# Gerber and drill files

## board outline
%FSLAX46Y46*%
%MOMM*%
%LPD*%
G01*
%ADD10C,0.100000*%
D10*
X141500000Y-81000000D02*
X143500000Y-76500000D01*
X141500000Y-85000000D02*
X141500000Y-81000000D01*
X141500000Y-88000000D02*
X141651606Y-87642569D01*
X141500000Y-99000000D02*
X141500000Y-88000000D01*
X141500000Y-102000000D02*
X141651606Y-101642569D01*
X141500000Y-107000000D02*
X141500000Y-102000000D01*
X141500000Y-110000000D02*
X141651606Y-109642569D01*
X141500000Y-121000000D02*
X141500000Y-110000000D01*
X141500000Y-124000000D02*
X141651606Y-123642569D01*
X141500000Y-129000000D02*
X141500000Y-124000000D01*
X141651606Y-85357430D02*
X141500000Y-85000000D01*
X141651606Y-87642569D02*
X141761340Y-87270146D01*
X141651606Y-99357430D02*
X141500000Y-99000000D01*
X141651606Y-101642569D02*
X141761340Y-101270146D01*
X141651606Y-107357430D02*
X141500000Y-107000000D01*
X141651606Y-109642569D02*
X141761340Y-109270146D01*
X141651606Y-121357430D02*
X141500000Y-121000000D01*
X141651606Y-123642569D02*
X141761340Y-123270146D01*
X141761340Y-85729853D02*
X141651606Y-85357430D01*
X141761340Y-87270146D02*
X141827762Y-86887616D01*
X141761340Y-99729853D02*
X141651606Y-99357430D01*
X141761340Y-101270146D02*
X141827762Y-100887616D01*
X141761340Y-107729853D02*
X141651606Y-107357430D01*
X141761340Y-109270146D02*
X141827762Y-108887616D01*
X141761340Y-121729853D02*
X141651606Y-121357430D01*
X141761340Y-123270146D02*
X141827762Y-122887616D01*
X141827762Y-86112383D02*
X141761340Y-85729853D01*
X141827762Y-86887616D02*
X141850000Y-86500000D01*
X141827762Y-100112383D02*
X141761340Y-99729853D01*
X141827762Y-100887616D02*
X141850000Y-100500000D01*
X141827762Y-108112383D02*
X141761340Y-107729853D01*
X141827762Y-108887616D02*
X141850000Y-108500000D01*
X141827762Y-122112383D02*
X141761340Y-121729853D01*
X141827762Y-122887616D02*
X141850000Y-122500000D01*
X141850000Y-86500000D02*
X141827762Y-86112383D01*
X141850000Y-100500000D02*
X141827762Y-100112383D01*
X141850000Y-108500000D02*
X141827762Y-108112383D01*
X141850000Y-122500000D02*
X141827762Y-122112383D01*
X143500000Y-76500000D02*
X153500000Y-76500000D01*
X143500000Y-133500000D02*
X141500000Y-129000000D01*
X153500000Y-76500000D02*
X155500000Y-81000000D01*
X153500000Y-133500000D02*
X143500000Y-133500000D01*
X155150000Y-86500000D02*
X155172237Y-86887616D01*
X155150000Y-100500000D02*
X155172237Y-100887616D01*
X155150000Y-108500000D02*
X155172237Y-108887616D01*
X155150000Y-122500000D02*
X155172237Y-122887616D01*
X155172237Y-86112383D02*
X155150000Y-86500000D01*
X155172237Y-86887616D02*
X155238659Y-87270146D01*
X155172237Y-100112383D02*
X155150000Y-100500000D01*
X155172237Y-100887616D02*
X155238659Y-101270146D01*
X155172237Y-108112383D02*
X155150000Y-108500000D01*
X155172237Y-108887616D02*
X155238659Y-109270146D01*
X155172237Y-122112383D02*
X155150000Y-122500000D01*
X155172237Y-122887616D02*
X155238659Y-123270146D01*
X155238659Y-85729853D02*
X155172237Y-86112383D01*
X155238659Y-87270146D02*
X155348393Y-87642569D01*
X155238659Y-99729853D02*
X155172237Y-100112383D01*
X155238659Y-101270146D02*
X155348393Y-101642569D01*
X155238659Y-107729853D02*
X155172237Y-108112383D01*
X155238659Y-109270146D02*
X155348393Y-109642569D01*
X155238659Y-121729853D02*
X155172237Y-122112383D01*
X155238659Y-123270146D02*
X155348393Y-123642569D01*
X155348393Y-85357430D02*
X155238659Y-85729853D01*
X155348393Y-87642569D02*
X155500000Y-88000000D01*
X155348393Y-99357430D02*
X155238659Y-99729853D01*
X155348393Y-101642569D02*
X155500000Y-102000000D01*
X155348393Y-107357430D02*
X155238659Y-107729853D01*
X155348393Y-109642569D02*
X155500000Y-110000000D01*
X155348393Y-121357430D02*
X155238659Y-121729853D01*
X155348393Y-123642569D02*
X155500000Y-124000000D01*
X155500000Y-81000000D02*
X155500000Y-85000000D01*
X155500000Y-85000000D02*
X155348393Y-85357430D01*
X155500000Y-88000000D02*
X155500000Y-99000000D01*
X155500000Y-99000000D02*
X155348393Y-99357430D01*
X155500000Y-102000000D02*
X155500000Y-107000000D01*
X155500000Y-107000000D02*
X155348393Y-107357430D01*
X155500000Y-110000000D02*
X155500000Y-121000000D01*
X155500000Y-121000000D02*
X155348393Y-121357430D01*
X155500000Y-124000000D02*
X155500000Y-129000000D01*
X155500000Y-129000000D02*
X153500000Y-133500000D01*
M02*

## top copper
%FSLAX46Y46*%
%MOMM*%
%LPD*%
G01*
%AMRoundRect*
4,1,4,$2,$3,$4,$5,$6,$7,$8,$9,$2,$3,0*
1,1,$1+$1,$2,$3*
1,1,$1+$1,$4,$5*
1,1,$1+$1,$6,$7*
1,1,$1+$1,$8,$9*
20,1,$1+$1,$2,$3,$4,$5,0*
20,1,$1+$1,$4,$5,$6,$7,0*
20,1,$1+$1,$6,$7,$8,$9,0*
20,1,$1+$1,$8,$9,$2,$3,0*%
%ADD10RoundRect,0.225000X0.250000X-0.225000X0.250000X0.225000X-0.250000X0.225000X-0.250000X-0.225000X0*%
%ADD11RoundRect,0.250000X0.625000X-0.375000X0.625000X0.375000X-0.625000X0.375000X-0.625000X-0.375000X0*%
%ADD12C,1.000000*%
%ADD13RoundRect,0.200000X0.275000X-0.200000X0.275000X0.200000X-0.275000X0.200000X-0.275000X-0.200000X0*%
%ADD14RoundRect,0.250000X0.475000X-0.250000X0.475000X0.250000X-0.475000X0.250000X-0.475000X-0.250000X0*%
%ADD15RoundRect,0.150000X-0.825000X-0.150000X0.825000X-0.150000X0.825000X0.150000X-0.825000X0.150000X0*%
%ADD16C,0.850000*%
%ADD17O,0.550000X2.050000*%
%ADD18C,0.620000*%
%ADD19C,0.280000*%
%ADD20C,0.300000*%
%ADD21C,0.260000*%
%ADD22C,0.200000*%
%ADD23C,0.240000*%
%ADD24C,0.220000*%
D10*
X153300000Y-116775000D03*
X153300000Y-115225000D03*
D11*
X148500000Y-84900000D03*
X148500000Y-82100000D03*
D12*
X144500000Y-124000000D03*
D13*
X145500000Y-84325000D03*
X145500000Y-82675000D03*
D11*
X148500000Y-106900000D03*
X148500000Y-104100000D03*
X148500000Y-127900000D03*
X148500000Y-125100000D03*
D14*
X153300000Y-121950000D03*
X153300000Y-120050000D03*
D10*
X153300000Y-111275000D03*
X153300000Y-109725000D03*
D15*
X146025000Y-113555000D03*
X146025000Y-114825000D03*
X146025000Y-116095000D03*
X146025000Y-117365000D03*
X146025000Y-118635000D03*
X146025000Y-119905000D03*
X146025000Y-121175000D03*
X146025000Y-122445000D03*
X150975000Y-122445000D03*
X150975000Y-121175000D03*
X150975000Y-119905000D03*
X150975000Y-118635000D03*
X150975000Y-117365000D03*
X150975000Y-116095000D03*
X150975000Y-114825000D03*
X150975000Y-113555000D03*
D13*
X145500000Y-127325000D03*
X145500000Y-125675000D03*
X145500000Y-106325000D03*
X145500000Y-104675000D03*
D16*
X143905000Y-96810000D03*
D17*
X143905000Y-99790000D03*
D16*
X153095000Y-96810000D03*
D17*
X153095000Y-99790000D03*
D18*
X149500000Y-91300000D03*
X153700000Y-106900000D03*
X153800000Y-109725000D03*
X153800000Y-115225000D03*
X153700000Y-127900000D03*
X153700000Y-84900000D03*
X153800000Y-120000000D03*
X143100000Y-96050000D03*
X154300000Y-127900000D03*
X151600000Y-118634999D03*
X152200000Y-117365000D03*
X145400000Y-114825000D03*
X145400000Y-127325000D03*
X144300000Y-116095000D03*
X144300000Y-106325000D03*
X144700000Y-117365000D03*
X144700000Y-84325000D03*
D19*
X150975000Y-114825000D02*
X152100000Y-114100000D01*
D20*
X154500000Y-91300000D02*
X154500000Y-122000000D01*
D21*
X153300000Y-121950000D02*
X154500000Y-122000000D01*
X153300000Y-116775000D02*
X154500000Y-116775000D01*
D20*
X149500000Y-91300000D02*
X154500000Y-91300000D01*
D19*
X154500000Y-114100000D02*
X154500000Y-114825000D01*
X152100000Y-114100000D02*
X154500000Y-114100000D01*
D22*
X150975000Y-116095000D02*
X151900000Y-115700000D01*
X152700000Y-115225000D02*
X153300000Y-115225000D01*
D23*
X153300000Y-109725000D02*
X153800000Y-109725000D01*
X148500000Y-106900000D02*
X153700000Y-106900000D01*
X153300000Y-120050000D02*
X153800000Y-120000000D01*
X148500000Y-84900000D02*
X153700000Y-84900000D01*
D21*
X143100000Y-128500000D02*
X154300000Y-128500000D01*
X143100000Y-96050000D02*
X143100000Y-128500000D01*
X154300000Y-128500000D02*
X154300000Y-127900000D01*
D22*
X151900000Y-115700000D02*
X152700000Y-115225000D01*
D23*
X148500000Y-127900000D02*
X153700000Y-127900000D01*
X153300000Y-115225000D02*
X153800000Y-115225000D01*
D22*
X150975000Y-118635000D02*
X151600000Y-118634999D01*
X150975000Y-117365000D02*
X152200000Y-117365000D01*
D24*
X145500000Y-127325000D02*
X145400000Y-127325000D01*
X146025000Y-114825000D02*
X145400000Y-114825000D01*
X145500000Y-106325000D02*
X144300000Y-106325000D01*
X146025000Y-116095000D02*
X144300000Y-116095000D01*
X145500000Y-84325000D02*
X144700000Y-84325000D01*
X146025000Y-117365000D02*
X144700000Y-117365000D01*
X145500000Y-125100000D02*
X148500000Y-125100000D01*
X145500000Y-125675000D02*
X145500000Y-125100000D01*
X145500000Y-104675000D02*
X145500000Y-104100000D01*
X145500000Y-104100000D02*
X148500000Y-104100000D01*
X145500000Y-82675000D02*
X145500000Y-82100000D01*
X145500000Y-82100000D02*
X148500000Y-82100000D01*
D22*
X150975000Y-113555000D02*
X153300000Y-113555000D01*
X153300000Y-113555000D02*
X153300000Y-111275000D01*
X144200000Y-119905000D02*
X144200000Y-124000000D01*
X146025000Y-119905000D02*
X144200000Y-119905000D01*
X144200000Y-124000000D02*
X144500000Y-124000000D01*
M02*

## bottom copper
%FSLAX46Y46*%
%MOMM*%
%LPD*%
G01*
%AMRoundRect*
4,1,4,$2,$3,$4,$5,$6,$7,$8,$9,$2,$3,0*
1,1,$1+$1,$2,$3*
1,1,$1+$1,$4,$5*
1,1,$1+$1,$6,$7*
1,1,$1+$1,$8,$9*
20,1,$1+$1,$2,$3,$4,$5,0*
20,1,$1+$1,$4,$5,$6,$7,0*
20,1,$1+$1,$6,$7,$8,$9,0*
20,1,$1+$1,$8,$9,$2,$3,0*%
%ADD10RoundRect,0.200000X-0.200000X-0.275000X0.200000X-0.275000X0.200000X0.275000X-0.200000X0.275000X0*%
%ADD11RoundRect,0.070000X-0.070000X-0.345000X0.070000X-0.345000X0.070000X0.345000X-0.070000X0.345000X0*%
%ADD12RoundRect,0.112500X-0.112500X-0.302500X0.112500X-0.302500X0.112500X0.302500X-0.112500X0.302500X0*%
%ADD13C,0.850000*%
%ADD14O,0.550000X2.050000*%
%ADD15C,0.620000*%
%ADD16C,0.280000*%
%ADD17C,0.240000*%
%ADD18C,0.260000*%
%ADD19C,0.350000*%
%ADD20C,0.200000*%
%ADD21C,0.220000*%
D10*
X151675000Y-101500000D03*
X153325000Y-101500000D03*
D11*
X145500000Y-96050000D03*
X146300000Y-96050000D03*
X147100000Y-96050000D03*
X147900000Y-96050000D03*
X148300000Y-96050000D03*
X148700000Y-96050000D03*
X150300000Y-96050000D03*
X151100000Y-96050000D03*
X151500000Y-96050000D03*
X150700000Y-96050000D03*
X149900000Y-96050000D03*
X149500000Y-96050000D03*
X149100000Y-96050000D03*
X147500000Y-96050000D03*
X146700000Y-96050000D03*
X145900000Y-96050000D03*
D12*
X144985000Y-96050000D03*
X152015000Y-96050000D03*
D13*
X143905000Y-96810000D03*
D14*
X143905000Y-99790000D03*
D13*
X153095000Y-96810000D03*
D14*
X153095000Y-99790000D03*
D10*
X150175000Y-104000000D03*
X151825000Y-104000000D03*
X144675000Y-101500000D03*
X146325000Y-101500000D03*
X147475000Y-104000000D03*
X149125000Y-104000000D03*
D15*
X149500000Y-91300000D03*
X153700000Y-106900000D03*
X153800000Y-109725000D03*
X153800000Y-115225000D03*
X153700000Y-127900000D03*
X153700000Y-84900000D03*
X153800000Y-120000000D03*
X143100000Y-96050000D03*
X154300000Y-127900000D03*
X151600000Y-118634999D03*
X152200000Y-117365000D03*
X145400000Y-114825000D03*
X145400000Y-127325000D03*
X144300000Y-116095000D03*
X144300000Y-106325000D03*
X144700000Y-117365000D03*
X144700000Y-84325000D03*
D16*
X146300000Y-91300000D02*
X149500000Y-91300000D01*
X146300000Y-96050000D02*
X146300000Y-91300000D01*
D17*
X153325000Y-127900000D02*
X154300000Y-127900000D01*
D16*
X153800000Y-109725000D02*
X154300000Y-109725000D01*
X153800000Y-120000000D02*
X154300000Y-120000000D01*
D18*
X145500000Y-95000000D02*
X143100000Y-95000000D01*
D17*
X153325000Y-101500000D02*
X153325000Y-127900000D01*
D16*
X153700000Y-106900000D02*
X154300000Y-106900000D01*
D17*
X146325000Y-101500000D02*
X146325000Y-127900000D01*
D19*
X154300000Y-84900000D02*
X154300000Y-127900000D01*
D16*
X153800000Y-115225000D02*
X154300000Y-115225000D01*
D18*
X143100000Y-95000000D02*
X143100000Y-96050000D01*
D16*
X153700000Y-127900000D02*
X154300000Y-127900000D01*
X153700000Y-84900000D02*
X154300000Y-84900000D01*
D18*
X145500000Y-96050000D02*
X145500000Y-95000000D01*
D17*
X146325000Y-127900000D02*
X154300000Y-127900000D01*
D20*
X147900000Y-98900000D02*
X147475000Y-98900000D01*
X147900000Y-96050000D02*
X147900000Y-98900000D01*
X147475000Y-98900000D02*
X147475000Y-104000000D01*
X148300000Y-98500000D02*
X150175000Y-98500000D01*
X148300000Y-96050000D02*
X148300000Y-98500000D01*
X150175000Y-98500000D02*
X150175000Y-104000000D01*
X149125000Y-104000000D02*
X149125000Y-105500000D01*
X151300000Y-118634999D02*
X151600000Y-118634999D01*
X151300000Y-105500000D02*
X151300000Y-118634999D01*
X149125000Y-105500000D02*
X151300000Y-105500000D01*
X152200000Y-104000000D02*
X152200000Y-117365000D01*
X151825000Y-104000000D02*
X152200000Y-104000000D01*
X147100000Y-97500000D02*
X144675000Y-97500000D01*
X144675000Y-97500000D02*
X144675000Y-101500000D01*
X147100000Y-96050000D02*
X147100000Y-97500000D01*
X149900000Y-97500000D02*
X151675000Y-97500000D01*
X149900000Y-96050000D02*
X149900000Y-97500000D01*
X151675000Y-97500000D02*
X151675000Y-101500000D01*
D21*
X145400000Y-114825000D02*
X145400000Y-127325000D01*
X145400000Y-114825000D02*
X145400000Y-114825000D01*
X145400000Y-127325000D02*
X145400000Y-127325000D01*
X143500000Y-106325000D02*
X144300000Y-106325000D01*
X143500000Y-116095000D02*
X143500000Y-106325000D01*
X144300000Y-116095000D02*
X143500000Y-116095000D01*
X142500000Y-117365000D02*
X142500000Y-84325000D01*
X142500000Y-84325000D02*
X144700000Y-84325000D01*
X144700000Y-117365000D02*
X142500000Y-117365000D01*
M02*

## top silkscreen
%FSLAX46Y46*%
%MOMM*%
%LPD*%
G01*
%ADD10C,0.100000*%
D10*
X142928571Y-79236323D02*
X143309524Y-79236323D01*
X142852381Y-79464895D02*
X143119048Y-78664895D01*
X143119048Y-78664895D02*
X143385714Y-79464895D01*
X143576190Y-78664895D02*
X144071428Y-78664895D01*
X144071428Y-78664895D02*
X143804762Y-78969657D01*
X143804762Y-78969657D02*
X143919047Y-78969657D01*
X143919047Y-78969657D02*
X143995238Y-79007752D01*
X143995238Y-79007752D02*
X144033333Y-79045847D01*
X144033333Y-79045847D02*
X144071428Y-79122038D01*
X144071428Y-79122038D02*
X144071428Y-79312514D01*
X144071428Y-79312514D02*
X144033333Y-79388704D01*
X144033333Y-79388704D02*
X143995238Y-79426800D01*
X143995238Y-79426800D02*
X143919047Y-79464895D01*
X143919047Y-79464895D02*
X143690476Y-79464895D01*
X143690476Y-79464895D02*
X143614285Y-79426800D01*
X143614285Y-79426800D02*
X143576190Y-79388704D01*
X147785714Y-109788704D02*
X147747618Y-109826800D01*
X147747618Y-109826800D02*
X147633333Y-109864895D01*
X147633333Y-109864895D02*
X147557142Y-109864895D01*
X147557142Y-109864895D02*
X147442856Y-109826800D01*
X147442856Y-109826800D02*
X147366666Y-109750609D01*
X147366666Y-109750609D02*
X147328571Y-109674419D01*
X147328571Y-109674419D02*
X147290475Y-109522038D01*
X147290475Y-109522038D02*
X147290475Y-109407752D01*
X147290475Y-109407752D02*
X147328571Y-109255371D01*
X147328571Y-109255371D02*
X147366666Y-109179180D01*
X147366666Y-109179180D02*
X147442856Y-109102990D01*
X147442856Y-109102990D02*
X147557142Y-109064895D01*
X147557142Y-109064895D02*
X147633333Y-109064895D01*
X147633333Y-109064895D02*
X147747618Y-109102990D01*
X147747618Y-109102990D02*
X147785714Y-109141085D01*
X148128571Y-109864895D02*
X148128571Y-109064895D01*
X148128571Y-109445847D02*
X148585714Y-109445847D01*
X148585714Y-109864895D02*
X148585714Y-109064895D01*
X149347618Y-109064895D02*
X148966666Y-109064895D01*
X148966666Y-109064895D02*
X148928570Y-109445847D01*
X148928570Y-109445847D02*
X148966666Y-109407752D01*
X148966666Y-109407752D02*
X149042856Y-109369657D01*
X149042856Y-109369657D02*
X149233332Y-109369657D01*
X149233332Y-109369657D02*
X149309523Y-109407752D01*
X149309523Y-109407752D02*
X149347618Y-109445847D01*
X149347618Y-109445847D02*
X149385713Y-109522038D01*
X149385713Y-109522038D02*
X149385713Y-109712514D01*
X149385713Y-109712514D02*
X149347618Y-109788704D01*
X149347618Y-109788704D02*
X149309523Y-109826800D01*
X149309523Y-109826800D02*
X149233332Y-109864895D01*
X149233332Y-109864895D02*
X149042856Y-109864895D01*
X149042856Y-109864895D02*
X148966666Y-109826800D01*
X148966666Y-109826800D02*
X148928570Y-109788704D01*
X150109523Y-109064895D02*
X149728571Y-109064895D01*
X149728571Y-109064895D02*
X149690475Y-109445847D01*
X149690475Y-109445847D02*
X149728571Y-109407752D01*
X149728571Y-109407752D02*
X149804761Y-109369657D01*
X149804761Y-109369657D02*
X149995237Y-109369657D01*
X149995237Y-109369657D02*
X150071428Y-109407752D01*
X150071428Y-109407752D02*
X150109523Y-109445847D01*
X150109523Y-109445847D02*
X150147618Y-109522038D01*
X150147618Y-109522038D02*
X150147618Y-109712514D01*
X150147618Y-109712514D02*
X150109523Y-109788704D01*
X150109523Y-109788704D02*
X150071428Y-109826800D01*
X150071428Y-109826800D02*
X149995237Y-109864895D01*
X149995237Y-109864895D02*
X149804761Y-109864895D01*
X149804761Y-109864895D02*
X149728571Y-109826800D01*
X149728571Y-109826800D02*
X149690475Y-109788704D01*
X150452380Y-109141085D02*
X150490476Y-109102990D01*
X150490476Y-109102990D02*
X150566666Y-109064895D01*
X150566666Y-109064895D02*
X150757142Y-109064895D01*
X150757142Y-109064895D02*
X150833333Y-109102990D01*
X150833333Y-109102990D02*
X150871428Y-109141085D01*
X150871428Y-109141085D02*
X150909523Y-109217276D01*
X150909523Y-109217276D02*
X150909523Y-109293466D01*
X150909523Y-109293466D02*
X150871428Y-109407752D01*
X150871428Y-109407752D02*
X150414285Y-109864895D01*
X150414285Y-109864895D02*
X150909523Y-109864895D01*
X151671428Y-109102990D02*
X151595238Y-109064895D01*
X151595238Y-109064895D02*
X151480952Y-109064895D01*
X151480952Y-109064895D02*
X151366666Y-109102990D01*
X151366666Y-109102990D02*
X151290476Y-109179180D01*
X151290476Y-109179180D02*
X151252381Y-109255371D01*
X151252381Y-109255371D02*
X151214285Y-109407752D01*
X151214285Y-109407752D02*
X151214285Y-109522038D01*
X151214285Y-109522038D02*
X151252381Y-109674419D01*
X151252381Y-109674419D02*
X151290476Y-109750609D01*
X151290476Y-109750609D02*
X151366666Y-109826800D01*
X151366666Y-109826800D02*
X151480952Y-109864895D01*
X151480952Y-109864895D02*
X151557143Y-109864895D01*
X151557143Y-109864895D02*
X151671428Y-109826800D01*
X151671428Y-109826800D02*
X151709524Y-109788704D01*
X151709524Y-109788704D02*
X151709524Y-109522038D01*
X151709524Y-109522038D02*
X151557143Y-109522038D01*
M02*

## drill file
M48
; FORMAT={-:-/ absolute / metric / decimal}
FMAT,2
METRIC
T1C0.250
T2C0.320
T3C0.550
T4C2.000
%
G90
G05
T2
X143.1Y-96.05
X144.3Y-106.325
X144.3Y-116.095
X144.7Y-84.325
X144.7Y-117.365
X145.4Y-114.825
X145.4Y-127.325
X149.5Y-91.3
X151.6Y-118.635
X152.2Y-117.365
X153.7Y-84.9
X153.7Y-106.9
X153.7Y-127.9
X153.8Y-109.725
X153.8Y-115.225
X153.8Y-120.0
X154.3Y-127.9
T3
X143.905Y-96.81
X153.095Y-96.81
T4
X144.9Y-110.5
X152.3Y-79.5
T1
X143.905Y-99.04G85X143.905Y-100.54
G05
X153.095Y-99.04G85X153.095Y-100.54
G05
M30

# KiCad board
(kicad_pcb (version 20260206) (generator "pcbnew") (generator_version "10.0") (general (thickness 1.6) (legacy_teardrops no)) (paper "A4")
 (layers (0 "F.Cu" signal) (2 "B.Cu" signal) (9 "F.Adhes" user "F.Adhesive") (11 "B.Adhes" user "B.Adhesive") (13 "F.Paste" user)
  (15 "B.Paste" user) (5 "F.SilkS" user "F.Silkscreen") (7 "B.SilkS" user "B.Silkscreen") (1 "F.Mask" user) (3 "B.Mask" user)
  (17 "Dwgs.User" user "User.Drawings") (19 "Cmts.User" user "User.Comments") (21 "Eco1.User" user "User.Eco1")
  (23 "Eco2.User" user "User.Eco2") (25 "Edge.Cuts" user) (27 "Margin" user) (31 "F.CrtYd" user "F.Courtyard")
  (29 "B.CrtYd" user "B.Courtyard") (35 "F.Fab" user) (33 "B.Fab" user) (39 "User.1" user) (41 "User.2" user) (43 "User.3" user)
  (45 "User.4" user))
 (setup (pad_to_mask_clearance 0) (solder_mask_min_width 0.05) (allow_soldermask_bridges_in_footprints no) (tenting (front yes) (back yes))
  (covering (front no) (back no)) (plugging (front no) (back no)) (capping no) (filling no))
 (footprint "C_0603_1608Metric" (layer "F.Cu") (at 153.3 116 90)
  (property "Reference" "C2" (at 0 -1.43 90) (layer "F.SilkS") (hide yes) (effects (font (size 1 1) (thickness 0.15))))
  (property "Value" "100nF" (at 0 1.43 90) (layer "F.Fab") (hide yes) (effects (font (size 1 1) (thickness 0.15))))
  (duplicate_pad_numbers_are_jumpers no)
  (pad "1" smd roundrect (at -0.775 0 90) (size 0.9 0.95) (layers "F.Cu" "F.Mask" "F.Paste") (roundrect_rratio 0.25) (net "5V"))
  (pad "2" smd roundrect (at 0.775 0 90) (size 0.9 0.95) (layers "F.Cu" "F.Mask" "F.Paste") (roundrect_rratio 0.25) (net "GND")))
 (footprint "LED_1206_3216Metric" (layer "F.Cu") (at 148.5 83.5 90)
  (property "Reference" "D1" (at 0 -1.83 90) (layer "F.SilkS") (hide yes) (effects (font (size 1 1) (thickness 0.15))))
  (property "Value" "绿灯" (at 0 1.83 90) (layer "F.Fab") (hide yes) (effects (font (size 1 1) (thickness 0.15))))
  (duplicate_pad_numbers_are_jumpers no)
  (pad "1" smd roundrect (at -1.4 0 90) (size 1.25 1.75) (layers "F.Cu" "F.Mask" "F.Paste") (roundrect_rratio 0.2) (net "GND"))
  (pad "2" smd roundrect (at 1.4 0 90) (size 1.25 1.75) (layers "F.Cu" "F.Mask" "F.Paste") (roundrect_rratio 0.2) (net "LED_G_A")))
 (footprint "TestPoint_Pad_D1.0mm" (layer "F.Cu") (at 144.5 124)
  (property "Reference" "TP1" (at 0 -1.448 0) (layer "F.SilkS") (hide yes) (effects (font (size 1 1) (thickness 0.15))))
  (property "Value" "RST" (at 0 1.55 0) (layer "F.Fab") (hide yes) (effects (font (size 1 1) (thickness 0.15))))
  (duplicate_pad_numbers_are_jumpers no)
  (pad "1" smd circle (at 0 0) (size 1 1) (layers "F.Cu" "F.Mask") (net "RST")))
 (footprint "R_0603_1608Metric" (layer "F.Cu") (at 145.5 83.5 90)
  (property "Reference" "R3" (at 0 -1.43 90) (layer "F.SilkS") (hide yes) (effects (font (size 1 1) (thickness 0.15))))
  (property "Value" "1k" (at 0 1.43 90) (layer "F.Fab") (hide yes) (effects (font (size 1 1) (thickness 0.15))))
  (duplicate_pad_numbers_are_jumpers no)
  (pad "1" smd roundrect (at -0.825 0 90) (size 0.8 0.95) (layers "F.Cu" "F.Mask" "F.Paste") (roundrect_rratio 0.25) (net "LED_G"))
  (pad "2" smd roundrect (at 0.825 0 90) (size 0.8 0.95) (layers "F.Cu" "F.Mask" "F.Paste") (roundrect_rratio 0.25) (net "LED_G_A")))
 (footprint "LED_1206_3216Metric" (layer "F.Cu") (at 148.5 105.5 90)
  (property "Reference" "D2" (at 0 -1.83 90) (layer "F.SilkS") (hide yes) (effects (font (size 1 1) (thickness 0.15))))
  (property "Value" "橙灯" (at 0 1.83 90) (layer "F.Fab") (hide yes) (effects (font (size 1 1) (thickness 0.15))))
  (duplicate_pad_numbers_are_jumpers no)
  (pad "1" smd roundrect (at -1.4 0 90) (size 1.25 1.75) (layers "F.Cu" "F.Mask" "F.Paste") (roundrect_rratio 0.2) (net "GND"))
  (pad "2" smd roundrect (at 1.4 0 90) (size 1.25 1.75) (layers "F.Cu" "F.Mask" "F.Paste") (roundrect_rratio 0.2) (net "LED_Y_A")))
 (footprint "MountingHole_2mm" (layer "F.Cu") (at 152.3 79.5)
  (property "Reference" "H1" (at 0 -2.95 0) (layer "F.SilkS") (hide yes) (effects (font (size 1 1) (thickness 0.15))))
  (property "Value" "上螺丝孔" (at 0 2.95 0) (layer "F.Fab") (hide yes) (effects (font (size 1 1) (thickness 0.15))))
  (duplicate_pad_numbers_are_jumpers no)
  (pad "" np_thru_hole circle (at 0 0) (size 2 2) (drill 2) (layers "*.Cu" "*.Mask")))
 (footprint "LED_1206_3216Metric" (layer "F.Cu") (at 148.5 126.5 90)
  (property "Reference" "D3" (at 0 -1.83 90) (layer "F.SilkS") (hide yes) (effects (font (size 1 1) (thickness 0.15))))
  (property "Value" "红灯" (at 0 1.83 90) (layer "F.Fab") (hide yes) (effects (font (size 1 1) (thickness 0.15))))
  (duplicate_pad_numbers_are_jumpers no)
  (pad "1" smd roundrect (at -1.4 0 90) (size 1.25 1.75) (layers "F.Cu" "F.Mask" "F.Paste") (roundrect_rratio 0.2) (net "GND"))
  (pad "2" smd roundrect (at 1.4 0 90) (size 1.25 1.75) (layers "F.Cu" "F.Mask" "F.Paste") (roundrect_rratio 0.2) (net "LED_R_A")))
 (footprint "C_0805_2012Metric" (layer "F.Cu") (at 153.3 121 90)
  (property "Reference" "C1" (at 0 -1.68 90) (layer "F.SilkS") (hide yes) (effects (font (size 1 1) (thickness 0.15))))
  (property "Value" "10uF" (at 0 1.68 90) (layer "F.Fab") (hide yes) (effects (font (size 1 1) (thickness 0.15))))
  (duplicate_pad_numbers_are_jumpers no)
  (pad "1" smd roundrect (at -0.95 0 90) (size 1 1.45) (layers "F.Cu" "F.Mask" "F.Paste") (roundrect_rratio 0.25) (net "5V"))
  (pad "2" smd roundrect (at 0.95 0 90) (size 1 1.45) (layers "F.Cu" "F.Mask" "F.Paste") (roundrect_rratio 0.25) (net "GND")))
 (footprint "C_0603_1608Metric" (layer "F.Cu") (at 153.3 110.5 90)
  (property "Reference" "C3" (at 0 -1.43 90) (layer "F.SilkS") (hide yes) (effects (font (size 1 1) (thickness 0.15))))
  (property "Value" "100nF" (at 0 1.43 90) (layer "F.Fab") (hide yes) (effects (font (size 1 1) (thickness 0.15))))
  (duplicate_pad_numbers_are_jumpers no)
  (pad "1" smd roundrect (at -0.775 0 90) (size 0.9 0.95) (layers "F.Cu" "F.Mask" "F.Paste") (roundrect_rratio 0.25) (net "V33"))
  (pad "2" smd roundrect (at 0.775 0 90) (size 0.9 0.95) (layers "F.Cu" "F.Mask" "F.Paste") (roundrect_rratio 0.25) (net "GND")))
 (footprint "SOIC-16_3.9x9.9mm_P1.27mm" (layer "F.Cu") (at 148.5 118)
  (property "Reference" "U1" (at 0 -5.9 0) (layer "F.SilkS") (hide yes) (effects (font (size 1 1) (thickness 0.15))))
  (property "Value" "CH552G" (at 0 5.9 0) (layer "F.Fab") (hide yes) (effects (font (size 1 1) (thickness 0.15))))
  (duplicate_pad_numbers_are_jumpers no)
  (pad "1" smd roundrect (at -2.475 -4.445) (size 1.95 0.6) (layers "F.Cu" "F.Mask" "F.Paste") (roundrect_rratio 0.25))
  (pad "2" smd roundrect (at -2.475 -3.175) (size 1.95 0.6) (layers "F.Cu" "F.Mask" "F.Paste") (roundrect_rratio 0.25) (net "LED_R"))
  (pad "3" smd roundrect (at -2.475 -1.905) (size 1.95 0.6) (layers "F.Cu" "F.Mask" "F.Paste") (roundrect_rratio 0.25) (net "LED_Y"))
  (pad "4" smd roundrect (at -2.475 -0.635) (size 1.95 0.6) (layers "F.Cu" "F.Mask" "F.Paste") (roundrect_rratio 0.25) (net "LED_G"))
  (pad "5" smd roundrect (at -2.475 0.635) (size 1.95 0.6) (layers "F.Cu" "F.Mask" "F.Paste") (roundrect_rratio 0.25))
  (pad "6" smd roundrect (at -2.475 1.905) (size 1.95 0.6) (layers "F.Cu" "F.Mask" "F.Paste") (roundrect_rratio 0.25) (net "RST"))
  (pad "7" smd roundrect (at -2.475 3.175) (size 1.95 0.6) (layers "F.Cu" "F.Mask" "F.Paste") (roundrect_rratio 0.25))
  (pad "8" smd roundrect (at -2.475 4.445) (size 1.95 0.6) (layers "F.Cu" "F.Mask" "F.Paste") (roundrect_rratio 0.25))
  (pad "9" smd roundrect (at 2.475 4.445) (size 1.95 0.6) (layers "F.Cu" "F.Mask" "F.Paste") (roundrect_rratio 0.25))
  (pad "10" smd roundrect (at 2.475 3.175) (size 1.95 0.6) (layers "F.Cu" "F.Mask" "F.Paste") (roundrect_rratio 0.25))
  (pad "11" smd roundrect (at 2.475 1.905) (size 1.95 0.6) (layers "F.Cu" "F.Mask" "F.Paste") (roundrect_rratio 0.25))
  (pad "12" smd roundrect (at 2.475 0.635) (size 1.95 0.6) (layers "F.Cu" "F.Mask" "F.Paste") (roundrect_rratio 0.25) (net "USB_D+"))
  (pad "13" smd roundrect (at 2.475 -0.635) (size 1.95 0.6) (layers "F.Cu" "F.Mask" "F.Paste") (roundrect_rratio 0.25) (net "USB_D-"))
  (pad "14" smd roundrect (at 2.475 -1.905) (size 1.95 0.6) (layers "F.Cu" "F.Mask" "F.Paste") (roundrect_rratio 0.25) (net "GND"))
  (pad "15" smd roundrect (at 2.475 -3.175) (size 1.95 0.6) (layers "F.Cu" "F.Mask" "F.Paste") (roundrect_rratio 0.25) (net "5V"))
  (pad "16" smd roundrect (at 2.475 -4.445) (size 1.95 0.6) (layers "F.Cu" "F.Mask" "F.Paste") (roundrect_rratio 0.25) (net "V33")))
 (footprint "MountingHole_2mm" (layer "F.Cu") (at 144.9 110.5)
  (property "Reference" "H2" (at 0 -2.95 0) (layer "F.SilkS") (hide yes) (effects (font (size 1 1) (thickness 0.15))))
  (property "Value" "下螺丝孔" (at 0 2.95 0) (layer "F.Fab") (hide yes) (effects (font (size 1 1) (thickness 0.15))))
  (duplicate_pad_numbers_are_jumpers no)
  (pad "" np_thru_hole circle (at 0 0) (size 2 2) (drill 2) (layers "*.Cu" "*.Mask")))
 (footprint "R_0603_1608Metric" (layer "F.Cu") (at 145.5 126.5 90)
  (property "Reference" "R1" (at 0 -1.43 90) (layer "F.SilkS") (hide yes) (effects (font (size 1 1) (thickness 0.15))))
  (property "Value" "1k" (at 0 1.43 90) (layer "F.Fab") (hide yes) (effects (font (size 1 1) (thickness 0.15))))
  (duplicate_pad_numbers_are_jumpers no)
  (pad "1" smd roundrect (at -0.825 0 90) (size 0.8 0.95) (layers "F.Cu" "F.Mask" "F.Paste") (roundrect_rratio 0.25) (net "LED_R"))
  (pad "2" smd roundrect (at 0.825 0 90) (size 0.8 0.95) (layers "F.Cu" "F.Mask" "F.Paste") (roundrect_rratio 0.25) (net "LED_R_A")))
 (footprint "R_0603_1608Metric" (layer "F.Cu") (at 145.5 105.5 90)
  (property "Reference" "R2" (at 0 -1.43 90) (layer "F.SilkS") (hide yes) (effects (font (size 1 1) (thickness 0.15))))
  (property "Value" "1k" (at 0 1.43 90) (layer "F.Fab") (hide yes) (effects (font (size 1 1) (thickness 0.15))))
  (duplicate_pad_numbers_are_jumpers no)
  (pad "1" smd roundrect (at -0.825 0 90) (size 0.8 0.95) (layers "F.Cu" "F.Mask" "F.Paste") (roundrect_rratio 0.25) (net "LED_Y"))
  (pad "2" smd roundrect (at 0.825 0 90) (size 0.8 0.95) (layers "F.Cu" "F.Mask" "F.Paste") (roundrect_rratio 0.25) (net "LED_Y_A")))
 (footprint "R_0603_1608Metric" (layer "B.Cu") (at 152.5 101.5)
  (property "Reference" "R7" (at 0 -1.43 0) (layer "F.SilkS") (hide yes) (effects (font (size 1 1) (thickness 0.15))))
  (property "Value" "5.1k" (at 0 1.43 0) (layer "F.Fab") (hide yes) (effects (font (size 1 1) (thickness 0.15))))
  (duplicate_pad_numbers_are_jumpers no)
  (pad "1" smd roundrect (at -0.825 0) (size 0.8 0.95) (layers "B.Cu" "B.Mask" "B.Paste") (roundrect_rratio 0.25) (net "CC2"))
  (pad "2" smd roundrect (at 0.825 0) (size 0.8 0.95) (layers "B.Cu" "B.Mask" "B.Paste") (roundrect_rratio 0.25) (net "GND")))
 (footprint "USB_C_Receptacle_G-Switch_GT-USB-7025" (layer "B.Cu") (at 148.5 99.5)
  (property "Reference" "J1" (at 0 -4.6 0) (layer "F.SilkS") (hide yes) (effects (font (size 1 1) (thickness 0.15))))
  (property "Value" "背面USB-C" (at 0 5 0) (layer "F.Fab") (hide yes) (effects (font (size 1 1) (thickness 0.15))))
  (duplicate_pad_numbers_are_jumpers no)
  (pad "A1" smd roundrect (at -3 -3.45) (size 0.28 0.83) (layers "B.Cu" "B.Mask" "B.Paste") (roundrect_rratio 0.25) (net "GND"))
  (pad "A4" smd roundrect (at -2.2 -3.45) (size 0.28 0.83) (layers "B.Cu" "B.Mask" "B.Paste") (roundrect_rratio 0.25) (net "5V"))
  (pad "A5" smd roundrect (at -1.4 -3.45) (size 0.28 0.83) (layers "B.Cu" "B.Mask" "B.Paste") (roundrect_rratio 0.25) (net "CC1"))
  (pad "A6" smd roundrect (at -0.6 -3.45) (size 0.28 0.83) (layers "B.Cu" "B.Mask" "B.Paste") (roundrect_rratio 0.25) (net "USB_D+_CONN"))
  (pad "A7" smd roundrect (at -0.2 -3.45) (size 0.28 0.83) (layers "B.Cu" "B.Mask" "B.Paste") (roundrect_rratio 0.25) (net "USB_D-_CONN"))
  (pad "A8" smd roundrect (at 0.2 -3.45) (size 0.28 0.83) (layers "B.Cu" "B.Mask" "B.Paste") (roundrect_rratio 0.25))
  (pad "A9" smd roundrect (at 1.8 -3.45) (size 0.28 0.83) (layers "B.Cu" "B.Mask" "B.Paste") (roundrect_rratio 0.25))
  (pad "A12" smd roundrect (at 2.6 -3.45) (size 0.28 0.83) (layers "B.Cu" "B.Mask" "B.Paste") (roundrect_rratio 0.25))
  (pad "B1" smd roundrect (at 3 -3.45) (size 0.28 0.83) (layers "B.Cu" "B.Mask" "B.Paste") (roundrect_rratio 0.25))
  (pad "B4" smd roundrect (at 2.2 -3.45) (size 0.28 0.83) (layers "B.Cu" "B.Mask" "B.Paste") (roundrect_rratio 0.25))
  (pad "B5" smd roundrect (at 1.4 -3.45) (size 0.28 0.83) (layers "B.Cu" "B.Mask" "B.Paste") (roundrect_rratio 0.25) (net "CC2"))
  (pad "B6" smd roundrect (at 1 -3.45) (size 0.28 0.83) (layers "B.Cu" "B.Mask" "B.Paste") (roundrect_rratio 0.25))
  (pad "B7" smd roundrect (at 0.6 -3.45) (size 0.28 0.83) (layers "B.Cu" "B.Mask" "B.Paste") (roundrect_rratio 0.25))
  (pad "B8" smd roundrect (at -1 -3.45) (size 0.28 0.83) (layers "B.Cu" "B.Mask" "B.Paste") (roundrect_rratio 0.25))
  (pad "B9" smd roundrect (at -1.8 -3.45) (size 0.28 0.83) (layers "B.Cu" "B.Mask" "B.Paste") (roundrect_rratio 0.25))
  (pad "B12" smd roundrect (at -2.6 -3.45) (size 0.28 0.83) (layers "B.Cu" "B.Mask" "B.Paste") (roundrect_rratio 0.25))
  (pad "GND" smd roundrect (at -3.515 -3.45) (size 0.45 0.83) (layers "B.Cu" "B.Mask" "B.Paste") (roundrect_rratio 0.25))
  (pad "GND" smd roundrect (at 3.515 -3.45) (size 0.45 0.83) (layers "B.Cu" "B.Mask" "B.Paste") (roundrect_rratio 0.25))
  (pad "SH" thru_hole circle (at -4.595 -2.69) (size 0.85 0.85) (drill 0.55) (layers "*.Cu" "*.Mask") (remove_unused_layers no))
  (pad "SH" thru_hole oval (at -4.595 0.29) (size 0.55 2.05) (drill oval 0.25 1.75) (layers "*.Cu" "*.Mask") (remove_unused_layers no))
  (pad "SH" thru_hole circle (at 4.595 -2.69) (size 0.85 0.85) (drill 0.55) (layers "*.Cu" "*.Mask") (remove_unused_layers no))
  (pad "SH" thru_hole oval (at 4.595 0.29) (size 0.55 2.05) (drill oval 0.25 1.75) (layers "*.Cu" "*.Mask") (remove_unused_layers no)))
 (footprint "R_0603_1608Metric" (layer "B.Cu") (at 151 104)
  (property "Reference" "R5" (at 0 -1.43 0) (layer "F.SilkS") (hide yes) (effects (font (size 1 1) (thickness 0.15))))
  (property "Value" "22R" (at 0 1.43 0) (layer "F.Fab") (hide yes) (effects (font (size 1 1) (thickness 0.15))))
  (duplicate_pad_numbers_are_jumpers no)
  (pad "1" smd roundrect (at -0.825 0) (size 0.8 0.95) (layers "B.Cu" "B.Mask" "B.Paste") (roundrect_rratio 0.25) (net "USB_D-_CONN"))
  (pad "2" smd roundrect (at 0.825 0) (size 0.8 0.95) (layers "B.Cu" "B.Mask" "B.Paste") (roundrect_rratio 0.25) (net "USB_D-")))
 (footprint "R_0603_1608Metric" (layer "B.Cu") (at 145.5 101.5)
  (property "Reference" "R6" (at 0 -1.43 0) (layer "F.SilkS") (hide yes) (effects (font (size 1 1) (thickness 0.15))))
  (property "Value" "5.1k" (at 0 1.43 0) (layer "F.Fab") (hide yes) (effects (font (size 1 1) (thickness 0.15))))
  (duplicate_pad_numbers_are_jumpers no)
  (pad "1" smd roundrect (at -0.825 0) (size 0.8 0.95) (layers "B.Cu" "B.Mask" "B.Paste") (roundrect_rratio 0.25) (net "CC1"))
  (pad "2" smd roundrect (at 0.825 0) (size 0.8 0.95) (layers "B.Cu" "B.Mask" "B.Paste") (roundrect_rratio 0.25) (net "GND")))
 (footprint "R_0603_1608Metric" (layer "B.Cu") (at 148.3 104)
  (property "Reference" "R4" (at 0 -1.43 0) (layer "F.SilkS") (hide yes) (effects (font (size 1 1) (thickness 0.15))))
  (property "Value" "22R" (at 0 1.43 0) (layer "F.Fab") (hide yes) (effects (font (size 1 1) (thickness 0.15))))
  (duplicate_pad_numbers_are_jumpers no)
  (pad "1" smd roundrect (at -0.825 0) (size 0.8 0.95) (layers "B.Cu" "B.Mask" "B.Paste") (roundrect_rratio 0.25) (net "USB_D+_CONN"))
  (pad "2" smd roundrect (at 0.825 0) (size 0.8 0.95) (layers "B.Cu" "B.Mask" "B.Paste") (roundrect_rratio 0.25) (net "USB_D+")))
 (gr_line (start 141.5 81) (end 143.5 76.5) (stroke (width 0.1) (type default)) (layer "Edge.Cuts"))
 (gr_line (start 141.5 85) (end 141.5 81) (stroke (width 0.1) (type default)) (layer "Edge.Cuts"))
 (gr_line (start 141.5 88) (end 141.651606 87.642569) (stroke (width 0.1) (type default)) (layer "Edge.Cuts"))
 (gr_line (start 141.5 99) (end 141.5 88) (stroke (width 0.1) (type default)) (layer "Edge.Cuts"))
 (gr_line (start 141.5 102) (end 141.651606 101.642569) (stroke (width 0.1) (type default)) (layer "Edge.Cuts"))
 (gr_line (start 141.5 107) (end 141.5 102) (stroke (width 0.1) (type default)) (layer "Edge.Cuts"))
 (gr_line (start 141.5 110) (end 141.651606 109.642569) (stroke (width 0.1) (type default)) (layer "Edge.Cuts"))
 (gr_line (start 141.5 121) (end 141.5 110) (stroke (width 0.1) (type default)) (layer "Edge.Cuts"))
 (gr_line (start 141.5 124) (end 141.651606 123.642569) (stroke (width 0.1) (type default)) (layer "Edge.Cuts"))
 (gr_line (start 141.5 129) (end 141.5 124) (stroke (width 0.1) (type default)) (layer "Edge.Cuts"))
 (gr_line (start 141.651606 85.35743) (end 141.5 85) (stroke (width 0.1) (type default)) (layer "Edge.Cuts"))
 (gr_line (start 141.651606 87.642569) (end 141.76134 87.270146) (stroke (width 0.1) (type default)) (layer "Edge.Cuts"))
 (gr_line (start 141.651606 99.35743) (end 141.5 99) (stroke (width 0.1) (type default)) (layer "Edge.Cuts"))
 (gr_line (start 141.651606 101.642569) (end 141.76134 101.270146) (stroke (width 0.1) (type default)) (layer "Edge.Cuts"))
 (gr_line (start 141.651606 107.35743) (end 141.5 107) (stroke (width 0.1) (type default)) (layer "Edge.Cuts"))
 (gr_line (start 141.651606 109.642569) (end 141.76134 109.270146) (stroke (width 0.1) (type default)) (layer "Edge.Cuts"))
 (gr_line (start 141.651606 121.35743) (end 141.5 121) (stroke (width 0.1) (type default)) (layer "Edge.Cuts"))
 (gr_line (start 141.651606 123.642569) (end 141.76134 123.270146) (stroke (width 0.1) (type default)) (layer "Edge.Cuts"))
 (gr_line (start 141.76134 85.729853) (end 141.651606 85.35743) (stroke (width 0.1) (type default)) (layer "Edge.Cuts"))
 (gr_line (start 141.76134 87.270146) (end 141.827762 86.887616) (stroke (width 0.1) (type default)) (layer "Edge.Cuts"))
 (gr_line (start 141.76134 99.729853) (end 141.651606 99.35743) (stroke (width 0.1) (type default)) (layer "Edge.Cuts"))
 (gr_line (start 141.76134 101.270146) (end 141.827762 100.887616) (stroke (width 0.1) (type default)) (layer "Edge.Cuts"))
 (gr_line (start 141.76134 107.729853) (end 141.651606 107.35743) (stroke (width 0.1) (type default)) (layer "Edge.Cuts"))
 (gr_line (start 141.76134 109.270146) (end 141.827762 108.887616) (stroke (width 0.1) (type default)) (layer "Edge.Cuts"))
 (gr_line (start 141.76134 121.729853) (end 141.651606 121.35743) (stroke (width 0.1) (type default)) (layer "Edge.Cuts"))
 (gr_line (start 141.76134 123.270146) (end 141.827762 122.887616) (stroke (width 0.1) (type default)) (layer "Edge.Cuts"))
 (gr_line (start 141.827762 86.112383) (end 141.76134 85.729853) (stroke (width 0.1) (type default)) (layer "Edge.Cuts"))
 (gr_line (start 141.827762 86.887616) (end 141.85 86.5) (stroke (width 0.1) (type default)) (layer "Edge.Cuts"))
 (gr_line (start 141.827762 100.112383) (end 141.76134 99.729853) (stroke (width 0.1) (type default)) (layer "Edge.Cuts"))
 (gr_line (start 141.827762 100.887616) (end 141.85 100.5) (stroke (width 0.1) (type default)) (layer "Edge.Cuts"))
 (gr_line (start 141.827762 108.112383) (end 141.76134 107.729853) (stroke (width 0.1) (type default)) (layer "Edge.Cuts"))
 (gr_line (start 141.827762 108.887616) (end 141.85 108.5) (stroke (width 0.1) (type default)) (layer "Edge.Cuts"))
 (gr_line (start 141.827762 122.112383) (end 141.76134 121.729853) (stroke (width 0.1) (type default)) (layer "Edge.Cuts"))
 (gr_line (start 141.827762 122.887616) (end 141.85 122.5) (stroke (width 0.1) (type default)) (layer "Edge.Cuts"))
 (gr_line (start 141.85 86.5) (end 141.827762 86.112383) (stroke (width 0.1) (type default)) (layer "Edge.Cuts"))
 (gr_line (start 141.85 100.5) (end 141.827762 100.112383) (stroke (width 0.1) (type default)) (layer "Edge.Cuts"))
 (gr_line (start 141.85 108.5) (end 141.827762 108.112383) (stroke (width 0.1) (type default)) (layer "Edge.Cuts"))
 (gr_line (start 141.85 122.5) (end 141.827762 122.112383) (stroke (width 0.1) (type default)) (layer "Edge.Cuts"))
 (gr_line (start 143.5 76.5) (end 153.5 76.5) (stroke (width 0.1) (type default)) (layer "Edge.Cuts"))
 (gr_line (start 143.5 133.5) (end 141.5 129) (stroke (width 0.1) (type default)) (layer "Edge.Cuts"))
 (gr_line (start 153.5 76.5) (end 155.5 81) (stroke (width 0.1) (type default)) (layer "Edge.Cuts"))
 (gr_line (start 153.5 133.5) (end 143.5 133.5) (stroke (width 0.1) (type default)) (layer "Edge.Cuts"))
 (gr_line (start 155.15 86.5) (end 155.172237 86.887616) (stroke (width 0.1) (type default)) (layer "Edge.Cuts"))
 (gr_line (start 155.15 100.5) (end 155.172237 100.887616) (stroke (width 0.1) (type default)) (layer "Edge.Cuts"))
 (gr_line (start 155.15 108.5) (end 155.172237 108.887616) (stroke (width 0.1) (type default)) (layer "Edge.Cuts"))
 (gr_line (start 155.15 122.5) (end 155.172237 122.887616) (stroke (width 0.1) (type default)) (layer "Edge.Cuts"))
 (gr_line (start 155.172237 86.112383) (end 155.15 86.5) (stroke (width 0.1) (type default)) (layer "Edge.Cuts"))
 (gr_line (start 155.172237 86.887616) (end 155.238659 87.270146) (stroke (width 0.1) (type default)) (layer "Edge.Cuts"))
 (gr_line (start 155.172237 100.112383) (end 155.15 100.5) (stroke (width 0.1) (type default)) (layer "Edge.Cuts"))
 (gr_line (start 155.172237 100.887616) (end 155.238659 101.270146) (stroke (width 0.1) (type default)) (layer "Edge.Cuts"))
 (gr_line (start 155.172237 108.112383) (end 155.15 108.5) (stroke (width 0.1) (type default)) (layer "Edge.Cuts"))
 (gr_line (start 155.172237 108.887616) (end 155.238659 109.270146) (stroke (width 0.1) (type default)) (layer "Edge.Cuts"))
 (gr_line (start 155.172237 122.112383) (end 155.15 122.5) (stroke (width 0.1) (type default)) (layer "Edge.Cuts"))
 (gr_line (start 155.172237 122.887616) (end 155.238659 123.270146) (stroke (width 0.1) (type default)) (layer "Edge.Cuts"))
 (gr_line (start 155.238659 85.729853) (end 155.172237 86.112383) (stroke (width 0.1) (type default)) (layer "Edge.Cuts"))
 (gr_line (start 155.238659 87.270146) (end 155.348393 87.642569) (stroke (width 0.1) (type default)) (layer "Edge.Cuts"))
 (gr_line (start 155.238659 99.729853) (end 155.172237 100.112383) (stroke (width 0.1) (type default)) (layer "Edge.Cuts"))
 (gr_line (start 155.238659 101.270146) (end 155.348393 101.642569) (stroke (width 0.1) (type default)) (layer "Edge.Cuts"))
 (gr_line (start 155.238659 107.729853) (end 155.172237 108.112383) (stroke (width 0.1) (type default)) (layer "Edge.Cuts"))
 (gr_line (start 155.238659 109.270146) (end 155.348393 109.642569) (stroke (width 0.1) (type default)) (layer "Edge.Cuts"))
 (gr_line (start 155.238659 121.729853) (end 155.172237 122.112383) (stroke (width 0.1) (type default)) (layer "Edge.Cuts"))
 (gr_line (start 155.238659 123.270146) (end 155.348393 123.642569) (stroke (width 0.1) (type default)) (layer "Edge.Cuts"))
 (gr_line (start 155.348393 85.35743) (end 155.238659 85.729853) (stroke (width 0.1) (type default)) (layer "Edge.Cuts"))
 (gr_line (start 155.348393 87.642569) (end 155.5 88) (stroke (width 0.1) (type default)) (layer "Edge.Cuts"))
 (gr_line (start 155.348393 99.35743) (end 155.238659 99.729853) (stroke (width 0.1) (type default)) (layer "Edge.Cuts"))
 (gr_line (start 155.348393 101.642569) (end 155.5 102) (stroke (width 0.1) (type default)) (layer "Edge.Cuts"))
 (gr_line (start 155.348393 107.35743) (end 155.238659 107.729853) (stroke (width 0.1) (type default)) (layer "Edge.Cuts"))
 (gr_line (start 155.348393 109.642569) (end 155.5 110) (stroke (width 0.1) (type default)) (layer "Edge.Cuts"))
 (gr_line (start 155.348393 121.35743) (end 155.238659 121.729853) (stroke (width 0.1) (type default)) (layer "Edge.Cuts"))
 (gr_line (start 155.348393 123.642569) (end 155.5 124) (stroke (width 0.1) (type default)) (layer "Edge.Cuts"))
 (gr_line (start 155.5 81) (end 155.5 85) (stroke (width 0.1) (type default)) (layer "Edge.Cuts"))
 (gr_line (start 155.5 85) (end 155.348393 85.35743) (stroke (width 0.1) (type default)) (layer "Edge.Cuts"))
 (gr_line (start 155.5 88) (end 155.5 99) (stroke (width 0.1) (type default)) (layer "Edge.Cuts"))
 (gr_line (start 155.5 99) (end 155.348393 99.35743) (stroke (width 0.1) (type default)) (layer "Edge.Cuts"))
 (gr_line (start 155.5 102) (end 155.5 107) (stroke (width 0.1) (type default)) (layer "Edge.Cuts"))
 (gr_line (start 155.5 107) (end 155.348393 107.35743) (stroke (width 0.1) (type default)) (layer "Edge.Cuts"))
 (gr_line (start 155.5 110) (end 155.5 121) (stroke (width 0.1) (type default)) (layer "Edge.Cuts"))
 (gr_line (start 155.5 121) (end 155.348393 121.35743) (stroke (width 0.1) (type default)) (layer "Edge.Cuts"))
 (gr_line (start 155.5 124) (end 155.5 129) (stroke (width 0.1) (type default)) (layer "Edge.Cuts"))
 (gr_line (start 155.5 129) (end 153.5 133.5) (stroke (width 0.1) (type default)) (layer "Edge.Cuts"))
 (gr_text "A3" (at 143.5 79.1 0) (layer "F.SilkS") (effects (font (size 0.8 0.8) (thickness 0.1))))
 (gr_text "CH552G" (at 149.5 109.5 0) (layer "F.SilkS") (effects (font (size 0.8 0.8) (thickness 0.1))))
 (segment (start 150.975 114.825) (end 152.1 114.1) (width 0.28) (layer "F.Cu") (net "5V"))
 (segment (start 154.5 91.3) (end 154.5 122) (width 0.3) (layer "F.Cu") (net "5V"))
 (segment (start 153.3 121.95) (end 154.5 122) (width 0.26) (layer "F.Cu") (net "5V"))
 (segment (start 153.3 116.775) (end 154.5 116.775) (width 0.26) (layer "F.Cu") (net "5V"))
 (segment (start 149.5 91.3) (end 154.5 91.3) (width 0.3) (layer "F.Cu") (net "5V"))
 (segment (start 154.5 114.1) (end 154.5 114.825) (width 0.28) (layer "F.Cu") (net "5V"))
 (segment (start 152.1 114.1) (end 154.5 114.1) (width 0.28) (layer "F.Cu") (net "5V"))
 (via (at 149.5 91.3) (size 0.62) (drill 0.32) (layers "F.Cu" "B.Cu") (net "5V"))
 (segment (start 146.3 91.3) (end 149.5 91.3) (width 0.28) (layer "B.Cu") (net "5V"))
 (segment (start 146.3 96.05) (end 146.3 91.3) (width 0.28) (layer "B.Cu") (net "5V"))
 (segment (start 150.975 116.095) (end 151.9 115.7) (width 0.2) (layer "F.Cu") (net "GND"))
 (segment (start 152.7 115.225) (end 153.3 115.225) (width 0.2) (layer "F.Cu") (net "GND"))
 (segment (start 153.3 109.725) (end 153.8 109.725) (width 0.24) (layer "F.Cu") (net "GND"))
 (segment (start 148.5 106.9) (end 153.7 106.9) (width 0.24) (layer "F.Cu") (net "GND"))
 (segment (start 153.3 120.05) (end 153.8 120) (width 0.24) (layer "F.Cu") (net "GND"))
 (segment (start 148.5 84.9) (end 153.7 84.9) (width 0.24) (layer "F.Cu") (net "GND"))
 (segment (start 143.1 128.5) (end 154.3 128.5) (width 0.26) (layer "F.Cu") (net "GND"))
 (segment (start 143.1 96.05) (end 143.1 128.5) (width 0.26) (layer "F.Cu") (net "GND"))
 (segment (start 154.3 128.5) (end 154.3 127.9) (width 0.26) (layer "F.Cu") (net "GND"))
 (segment (start 151.9 115.7) (end 152.7 115.225) (width 0.2) (layer "F.Cu") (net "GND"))
 (segment (start 148.5 127.9) (end 153.7 127.9) (width 0.24) (layer "F.Cu") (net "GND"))
 (segment (start 153.3 115.225) (end 153.8 115.225) (width 0.24) (layer "F.Cu") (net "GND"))
 (via (at 153.7 106.9) (size 0.62) (drill 0.32) (layers "F.Cu" "B.Cu") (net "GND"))
 (via (at 153.8 109.725) (size 0.62) (drill 0.32) (layers "F.Cu" "B.Cu") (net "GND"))
 (via (at 153.8 115.225) (size 0.62) (drill 0.32) (layers "F.Cu" "B.Cu") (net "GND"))
 (via (at 153.7 127.9) (size 0.62) (drill 0.32) (layers "F.Cu" "B.Cu") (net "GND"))
 (via (at 153.7 84.9) (size 0.62) (drill 0.32) (layers "F.Cu" "B.Cu") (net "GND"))
 (via (at 153.8 120) (size 0.62) (drill 0.32) (layers "F.Cu" "B.Cu") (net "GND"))
 (via (at 143.1 96.05) (size 0.62) (drill 0.32) (layers "F.Cu" "B.Cu") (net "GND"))
 (via (at 154.3 127.9) (size 0.62) (drill 0.32) (layers "F.Cu" "B.Cu") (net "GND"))
 (segment (start 153.325 127.9) (end 154.3 127.9) (width 0.24) (layer "B.Cu") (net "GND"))
 (segment (start 153.8 109.725) (end 154.3 109.725) (width 0.28) (layer "B.Cu") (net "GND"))
 (segment (start 153.8 120) (end 154.3 120) (width 0.28) (layer "B.Cu") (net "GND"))
 (segment (start 145.5 95) (end 143.1 95) (width 0.26) (layer "B.Cu") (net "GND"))
 (segment (start 153.325 101.5) (end 153.325 127.9) (width 0.24) (layer "B.Cu") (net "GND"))
 (segment (start 153.7 106.9) (end 154.3 106.9) (width 0.28) (layer "B.Cu") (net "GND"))
 (segment (start 146.325 101.5) (end 146.325 127.9) (width 0.24) (layer "B.Cu") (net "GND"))
 (segment (start 154.3 84.9) (end 154.3 127.9) (width 0.35) (layer "B.Cu") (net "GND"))
 (segment (start 153.8 115.225) (end 154.3 115.225) (width 0.28) (layer "B.Cu") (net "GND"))
 (segment (start 143.1 95) (end 143.1 96.05) (width 0.26) (layer "B.Cu") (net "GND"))
 (segment (start 153.7 127.9) (end 154.3 127.9) (width 0.28) (layer "B.Cu") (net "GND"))
 (segment (start 153.7 84.9) (end 154.3 84.9) (width 0.28) (layer "B.Cu") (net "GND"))
 (segment (start 145.5 96.05) (end 145.5 95) (width 0.26) (layer "B.Cu") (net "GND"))
 (segment (start 146.325 127.9) (end 154.3 127.9) (width 0.24) (layer "B.Cu") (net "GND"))
 (segment (start 147.9 98.9) (end 147.475 98.9) (width 0.2) (layer "B.Cu") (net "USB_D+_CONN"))
 (segment (start 147.9 96.05) (end 147.9 98.9) (width 0.2) (layer "B.Cu") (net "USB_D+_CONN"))
 (segment (start 147.475 98.9) (end 147.475 104) (width 0.2) (layer "B.Cu") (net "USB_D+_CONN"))
 (segment (start 148.3 98.5) (end 150.175 98.5) (width 0.2) (layer "B.Cu") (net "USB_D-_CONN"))
 (segment (start 148.3 96.05) (end 148.3 98.5) (width 0.2) (layer "B.Cu") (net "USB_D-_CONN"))
 (segment (start 150.175 98.5) (end 150.175 104) (width 0.2) (layer "B.Cu") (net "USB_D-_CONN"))
 (segment (start 150.975 118.635) (end 151.6 118.634999) (width 0.2) (layer "F.Cu") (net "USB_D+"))
 (via (at 151.6 118.634999) (size 0.62) (drill 0.32) (layers "F.Cu" "B.Cu") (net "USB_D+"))
 (segment (start 149.125 104) (end 149.125 105.5) (width 0.2) (layer "B.Cu") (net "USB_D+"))
 (segment (start 151.3 118.634999) (end 151.6 118.634999) (width 0.2) (layer "B.Cu") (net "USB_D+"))
 (segment (start 151.3 105.5) (end 151.3 118.634999) (width 0.2) (layer "B.Cu") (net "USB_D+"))
 (segment (start 149.125 105.5) (end 151.3 105.5) (width 0.2) (layer "B.Cu") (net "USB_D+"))
 (segment (start 150.975 117.365) (end 152.2 117.365) (width 0.2) (layer "F.Cu") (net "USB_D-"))
 (via (at 152.2 117.365) (size 0.62) (drill 0.32) (layers "F.Cu" "B.Cu") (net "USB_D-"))
 (segment (start 152.2 104) (end 152.2 117.365) (width 0.2) (layer "B.Cu") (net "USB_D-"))
 (segment (start 151.825 104) (end 152.2 104) (width 0.2) (layer "B.Cu") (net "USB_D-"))
 (segment (start 147.1 97.5) (end 144.675 97.5) (width 0.2) (layer "B.Cu") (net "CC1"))
 (segment (start 144.675 97.5) (end 144.675 101.5) (width 0.2) (layer "B.Cu") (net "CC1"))
 (segment (start 147.1 96.05) (end 147.1 97.5) (width 0.2) (layer "B.Cu") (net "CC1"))
 (segment (start 149.9 97.5) (end 151.675 97.5) (width 0.2) (layer "B.Cu") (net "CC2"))
 (segment (start 149.9 96.05) (end 149.9 97.5) (width 0.2) (layer "B.Cu") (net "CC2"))
 (segment (start 151.675 97.5) (end 151.675 101.5) (width 0.2) (layer "B.Cu") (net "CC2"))
 (segment (start 145.5 127.325) (end 145.4 127.325) (width 0.22) (layer "F.Cu") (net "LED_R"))
 (segment (start 146.025 114.825) (end 145.4 114.825) (width 0.22) (layer "F.Cu") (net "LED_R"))
 (via (at 145.4 114.825) (size 0.62) (drill 0.32) (layers "F.Cu" "B.Cu") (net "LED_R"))
 (via (at 145.4 127.325) (size 0.62) (drill 0.32) (layers "F.Cu" "B.Cu") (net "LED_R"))
 (segment (start 145.4 114.825) (end 145.4 127.325) (width 0.22) (layer "B.Cu") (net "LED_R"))
 (segment (start 145.4 114.825) (end 145.4 114.825) (width 0.22) (layer "B.Cu") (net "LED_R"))
 (segment (start 145.4 127.325) (end 145.4 127.325) (width 0.22) (layer "B.Cu") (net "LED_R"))
 (segment (start 145.5 106.325) (end 144.3 106.325) (width 0.22) (layer "F.Cu") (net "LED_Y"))
 (segment (start 146.025 116.095) (end 144.3 116.095) (width 0.22) (layer "F.Cu") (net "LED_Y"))
 (via (at 144.3 116.095) (size 0.62) (drill 0.32) (layers "F.Cu" "B.Cu") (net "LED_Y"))
 (via (at 144.3 106.325) (size 0.62) (drill 0.32) (layers "F.Cu" "B.Cu") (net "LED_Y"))
 (segment (start 143.5 106.325) (end 144.3 106.325) (width 0.22) (layer "B.Cu") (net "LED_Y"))
 (segment (start 143.5 116.095) (end 143.5 106.325) (width 0.22) (layer "B.Cu") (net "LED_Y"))
 (segment (start 144.3 116.095) (end 143.5 116.095) (width 0.22) (layer "B.Cu") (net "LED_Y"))
 (segment (start 145.5 84.325) (end 144.7 84.325) (width 0.22) (layer "F.Cu") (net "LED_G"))
 (segment (start 146.025 117.365) (end 144.7 117.365) (width 0.22) (layer "F.Cu") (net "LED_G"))
 (via (at 144.7 117.365) (size 0.62) (drill 0.32) (layers "F.Cu" "B.Cu") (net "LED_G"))
 (via (at 144.7 84.325) (size 0.62) (drill 0.32) (layers "F.Cu" "B.Cu") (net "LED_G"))
 (segment (start 142.5 117.365) (end 142.5 84.325) (width 0.22) (layer "B.Cu") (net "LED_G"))
 (segment (start 142.5 84.325) (end 144.7 84.325) (width 0.22) (layer "B.Cu") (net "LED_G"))
 (segment (start 144.7 117.365) (end 142.5 117.365) (width 0.22) (layer "B.Cu") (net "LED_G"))
 (segment (start 145.5 125.1) (end 148.5 125.1) (width 0.22) (layer "F.Cu") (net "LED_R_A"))
 (segment (start 145.5 125.675) (end 145.5 125.1) (width 0.22) (layer "F.Cu") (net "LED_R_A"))
 (segment (start 145.5 104.675) (end 145.5 104.1) (width 0.22) (layer "F.Cu") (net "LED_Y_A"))
 (segment (start 145.5 104.1) (end 148.5 104.1) (width 0.22) (layer "F.Cu") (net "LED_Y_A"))
 (segment (start 145.5 82.675) (end 145.5 82.1) (width 0.22) (layer "F.Cu") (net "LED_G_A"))
 (segment (start 145.5 82.1) (end 148.5 82.1) (width 0.22) (layer "F.Cu") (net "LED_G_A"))
 (segment (start 150.975 113.555) (end 153.3 113.555) (width 0.2) (layer "F.Cu") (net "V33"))
 (segment (start 153.3 113.555) (end 153.3 111.275) (width 0.2) (layer "F.Cu") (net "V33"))
 (segment (start 144.2 119.905) (end 144.2 124) (width 0.2) (layer "F.Cu") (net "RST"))
 (segment (start 146.025 119.905) (end 144.2 119.905) (width 0.2) (layer "F.Cu") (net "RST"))
 (segment (start 144.2 124) (end 144.5 124) (width 0.2) (layer "F.Cu") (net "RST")))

